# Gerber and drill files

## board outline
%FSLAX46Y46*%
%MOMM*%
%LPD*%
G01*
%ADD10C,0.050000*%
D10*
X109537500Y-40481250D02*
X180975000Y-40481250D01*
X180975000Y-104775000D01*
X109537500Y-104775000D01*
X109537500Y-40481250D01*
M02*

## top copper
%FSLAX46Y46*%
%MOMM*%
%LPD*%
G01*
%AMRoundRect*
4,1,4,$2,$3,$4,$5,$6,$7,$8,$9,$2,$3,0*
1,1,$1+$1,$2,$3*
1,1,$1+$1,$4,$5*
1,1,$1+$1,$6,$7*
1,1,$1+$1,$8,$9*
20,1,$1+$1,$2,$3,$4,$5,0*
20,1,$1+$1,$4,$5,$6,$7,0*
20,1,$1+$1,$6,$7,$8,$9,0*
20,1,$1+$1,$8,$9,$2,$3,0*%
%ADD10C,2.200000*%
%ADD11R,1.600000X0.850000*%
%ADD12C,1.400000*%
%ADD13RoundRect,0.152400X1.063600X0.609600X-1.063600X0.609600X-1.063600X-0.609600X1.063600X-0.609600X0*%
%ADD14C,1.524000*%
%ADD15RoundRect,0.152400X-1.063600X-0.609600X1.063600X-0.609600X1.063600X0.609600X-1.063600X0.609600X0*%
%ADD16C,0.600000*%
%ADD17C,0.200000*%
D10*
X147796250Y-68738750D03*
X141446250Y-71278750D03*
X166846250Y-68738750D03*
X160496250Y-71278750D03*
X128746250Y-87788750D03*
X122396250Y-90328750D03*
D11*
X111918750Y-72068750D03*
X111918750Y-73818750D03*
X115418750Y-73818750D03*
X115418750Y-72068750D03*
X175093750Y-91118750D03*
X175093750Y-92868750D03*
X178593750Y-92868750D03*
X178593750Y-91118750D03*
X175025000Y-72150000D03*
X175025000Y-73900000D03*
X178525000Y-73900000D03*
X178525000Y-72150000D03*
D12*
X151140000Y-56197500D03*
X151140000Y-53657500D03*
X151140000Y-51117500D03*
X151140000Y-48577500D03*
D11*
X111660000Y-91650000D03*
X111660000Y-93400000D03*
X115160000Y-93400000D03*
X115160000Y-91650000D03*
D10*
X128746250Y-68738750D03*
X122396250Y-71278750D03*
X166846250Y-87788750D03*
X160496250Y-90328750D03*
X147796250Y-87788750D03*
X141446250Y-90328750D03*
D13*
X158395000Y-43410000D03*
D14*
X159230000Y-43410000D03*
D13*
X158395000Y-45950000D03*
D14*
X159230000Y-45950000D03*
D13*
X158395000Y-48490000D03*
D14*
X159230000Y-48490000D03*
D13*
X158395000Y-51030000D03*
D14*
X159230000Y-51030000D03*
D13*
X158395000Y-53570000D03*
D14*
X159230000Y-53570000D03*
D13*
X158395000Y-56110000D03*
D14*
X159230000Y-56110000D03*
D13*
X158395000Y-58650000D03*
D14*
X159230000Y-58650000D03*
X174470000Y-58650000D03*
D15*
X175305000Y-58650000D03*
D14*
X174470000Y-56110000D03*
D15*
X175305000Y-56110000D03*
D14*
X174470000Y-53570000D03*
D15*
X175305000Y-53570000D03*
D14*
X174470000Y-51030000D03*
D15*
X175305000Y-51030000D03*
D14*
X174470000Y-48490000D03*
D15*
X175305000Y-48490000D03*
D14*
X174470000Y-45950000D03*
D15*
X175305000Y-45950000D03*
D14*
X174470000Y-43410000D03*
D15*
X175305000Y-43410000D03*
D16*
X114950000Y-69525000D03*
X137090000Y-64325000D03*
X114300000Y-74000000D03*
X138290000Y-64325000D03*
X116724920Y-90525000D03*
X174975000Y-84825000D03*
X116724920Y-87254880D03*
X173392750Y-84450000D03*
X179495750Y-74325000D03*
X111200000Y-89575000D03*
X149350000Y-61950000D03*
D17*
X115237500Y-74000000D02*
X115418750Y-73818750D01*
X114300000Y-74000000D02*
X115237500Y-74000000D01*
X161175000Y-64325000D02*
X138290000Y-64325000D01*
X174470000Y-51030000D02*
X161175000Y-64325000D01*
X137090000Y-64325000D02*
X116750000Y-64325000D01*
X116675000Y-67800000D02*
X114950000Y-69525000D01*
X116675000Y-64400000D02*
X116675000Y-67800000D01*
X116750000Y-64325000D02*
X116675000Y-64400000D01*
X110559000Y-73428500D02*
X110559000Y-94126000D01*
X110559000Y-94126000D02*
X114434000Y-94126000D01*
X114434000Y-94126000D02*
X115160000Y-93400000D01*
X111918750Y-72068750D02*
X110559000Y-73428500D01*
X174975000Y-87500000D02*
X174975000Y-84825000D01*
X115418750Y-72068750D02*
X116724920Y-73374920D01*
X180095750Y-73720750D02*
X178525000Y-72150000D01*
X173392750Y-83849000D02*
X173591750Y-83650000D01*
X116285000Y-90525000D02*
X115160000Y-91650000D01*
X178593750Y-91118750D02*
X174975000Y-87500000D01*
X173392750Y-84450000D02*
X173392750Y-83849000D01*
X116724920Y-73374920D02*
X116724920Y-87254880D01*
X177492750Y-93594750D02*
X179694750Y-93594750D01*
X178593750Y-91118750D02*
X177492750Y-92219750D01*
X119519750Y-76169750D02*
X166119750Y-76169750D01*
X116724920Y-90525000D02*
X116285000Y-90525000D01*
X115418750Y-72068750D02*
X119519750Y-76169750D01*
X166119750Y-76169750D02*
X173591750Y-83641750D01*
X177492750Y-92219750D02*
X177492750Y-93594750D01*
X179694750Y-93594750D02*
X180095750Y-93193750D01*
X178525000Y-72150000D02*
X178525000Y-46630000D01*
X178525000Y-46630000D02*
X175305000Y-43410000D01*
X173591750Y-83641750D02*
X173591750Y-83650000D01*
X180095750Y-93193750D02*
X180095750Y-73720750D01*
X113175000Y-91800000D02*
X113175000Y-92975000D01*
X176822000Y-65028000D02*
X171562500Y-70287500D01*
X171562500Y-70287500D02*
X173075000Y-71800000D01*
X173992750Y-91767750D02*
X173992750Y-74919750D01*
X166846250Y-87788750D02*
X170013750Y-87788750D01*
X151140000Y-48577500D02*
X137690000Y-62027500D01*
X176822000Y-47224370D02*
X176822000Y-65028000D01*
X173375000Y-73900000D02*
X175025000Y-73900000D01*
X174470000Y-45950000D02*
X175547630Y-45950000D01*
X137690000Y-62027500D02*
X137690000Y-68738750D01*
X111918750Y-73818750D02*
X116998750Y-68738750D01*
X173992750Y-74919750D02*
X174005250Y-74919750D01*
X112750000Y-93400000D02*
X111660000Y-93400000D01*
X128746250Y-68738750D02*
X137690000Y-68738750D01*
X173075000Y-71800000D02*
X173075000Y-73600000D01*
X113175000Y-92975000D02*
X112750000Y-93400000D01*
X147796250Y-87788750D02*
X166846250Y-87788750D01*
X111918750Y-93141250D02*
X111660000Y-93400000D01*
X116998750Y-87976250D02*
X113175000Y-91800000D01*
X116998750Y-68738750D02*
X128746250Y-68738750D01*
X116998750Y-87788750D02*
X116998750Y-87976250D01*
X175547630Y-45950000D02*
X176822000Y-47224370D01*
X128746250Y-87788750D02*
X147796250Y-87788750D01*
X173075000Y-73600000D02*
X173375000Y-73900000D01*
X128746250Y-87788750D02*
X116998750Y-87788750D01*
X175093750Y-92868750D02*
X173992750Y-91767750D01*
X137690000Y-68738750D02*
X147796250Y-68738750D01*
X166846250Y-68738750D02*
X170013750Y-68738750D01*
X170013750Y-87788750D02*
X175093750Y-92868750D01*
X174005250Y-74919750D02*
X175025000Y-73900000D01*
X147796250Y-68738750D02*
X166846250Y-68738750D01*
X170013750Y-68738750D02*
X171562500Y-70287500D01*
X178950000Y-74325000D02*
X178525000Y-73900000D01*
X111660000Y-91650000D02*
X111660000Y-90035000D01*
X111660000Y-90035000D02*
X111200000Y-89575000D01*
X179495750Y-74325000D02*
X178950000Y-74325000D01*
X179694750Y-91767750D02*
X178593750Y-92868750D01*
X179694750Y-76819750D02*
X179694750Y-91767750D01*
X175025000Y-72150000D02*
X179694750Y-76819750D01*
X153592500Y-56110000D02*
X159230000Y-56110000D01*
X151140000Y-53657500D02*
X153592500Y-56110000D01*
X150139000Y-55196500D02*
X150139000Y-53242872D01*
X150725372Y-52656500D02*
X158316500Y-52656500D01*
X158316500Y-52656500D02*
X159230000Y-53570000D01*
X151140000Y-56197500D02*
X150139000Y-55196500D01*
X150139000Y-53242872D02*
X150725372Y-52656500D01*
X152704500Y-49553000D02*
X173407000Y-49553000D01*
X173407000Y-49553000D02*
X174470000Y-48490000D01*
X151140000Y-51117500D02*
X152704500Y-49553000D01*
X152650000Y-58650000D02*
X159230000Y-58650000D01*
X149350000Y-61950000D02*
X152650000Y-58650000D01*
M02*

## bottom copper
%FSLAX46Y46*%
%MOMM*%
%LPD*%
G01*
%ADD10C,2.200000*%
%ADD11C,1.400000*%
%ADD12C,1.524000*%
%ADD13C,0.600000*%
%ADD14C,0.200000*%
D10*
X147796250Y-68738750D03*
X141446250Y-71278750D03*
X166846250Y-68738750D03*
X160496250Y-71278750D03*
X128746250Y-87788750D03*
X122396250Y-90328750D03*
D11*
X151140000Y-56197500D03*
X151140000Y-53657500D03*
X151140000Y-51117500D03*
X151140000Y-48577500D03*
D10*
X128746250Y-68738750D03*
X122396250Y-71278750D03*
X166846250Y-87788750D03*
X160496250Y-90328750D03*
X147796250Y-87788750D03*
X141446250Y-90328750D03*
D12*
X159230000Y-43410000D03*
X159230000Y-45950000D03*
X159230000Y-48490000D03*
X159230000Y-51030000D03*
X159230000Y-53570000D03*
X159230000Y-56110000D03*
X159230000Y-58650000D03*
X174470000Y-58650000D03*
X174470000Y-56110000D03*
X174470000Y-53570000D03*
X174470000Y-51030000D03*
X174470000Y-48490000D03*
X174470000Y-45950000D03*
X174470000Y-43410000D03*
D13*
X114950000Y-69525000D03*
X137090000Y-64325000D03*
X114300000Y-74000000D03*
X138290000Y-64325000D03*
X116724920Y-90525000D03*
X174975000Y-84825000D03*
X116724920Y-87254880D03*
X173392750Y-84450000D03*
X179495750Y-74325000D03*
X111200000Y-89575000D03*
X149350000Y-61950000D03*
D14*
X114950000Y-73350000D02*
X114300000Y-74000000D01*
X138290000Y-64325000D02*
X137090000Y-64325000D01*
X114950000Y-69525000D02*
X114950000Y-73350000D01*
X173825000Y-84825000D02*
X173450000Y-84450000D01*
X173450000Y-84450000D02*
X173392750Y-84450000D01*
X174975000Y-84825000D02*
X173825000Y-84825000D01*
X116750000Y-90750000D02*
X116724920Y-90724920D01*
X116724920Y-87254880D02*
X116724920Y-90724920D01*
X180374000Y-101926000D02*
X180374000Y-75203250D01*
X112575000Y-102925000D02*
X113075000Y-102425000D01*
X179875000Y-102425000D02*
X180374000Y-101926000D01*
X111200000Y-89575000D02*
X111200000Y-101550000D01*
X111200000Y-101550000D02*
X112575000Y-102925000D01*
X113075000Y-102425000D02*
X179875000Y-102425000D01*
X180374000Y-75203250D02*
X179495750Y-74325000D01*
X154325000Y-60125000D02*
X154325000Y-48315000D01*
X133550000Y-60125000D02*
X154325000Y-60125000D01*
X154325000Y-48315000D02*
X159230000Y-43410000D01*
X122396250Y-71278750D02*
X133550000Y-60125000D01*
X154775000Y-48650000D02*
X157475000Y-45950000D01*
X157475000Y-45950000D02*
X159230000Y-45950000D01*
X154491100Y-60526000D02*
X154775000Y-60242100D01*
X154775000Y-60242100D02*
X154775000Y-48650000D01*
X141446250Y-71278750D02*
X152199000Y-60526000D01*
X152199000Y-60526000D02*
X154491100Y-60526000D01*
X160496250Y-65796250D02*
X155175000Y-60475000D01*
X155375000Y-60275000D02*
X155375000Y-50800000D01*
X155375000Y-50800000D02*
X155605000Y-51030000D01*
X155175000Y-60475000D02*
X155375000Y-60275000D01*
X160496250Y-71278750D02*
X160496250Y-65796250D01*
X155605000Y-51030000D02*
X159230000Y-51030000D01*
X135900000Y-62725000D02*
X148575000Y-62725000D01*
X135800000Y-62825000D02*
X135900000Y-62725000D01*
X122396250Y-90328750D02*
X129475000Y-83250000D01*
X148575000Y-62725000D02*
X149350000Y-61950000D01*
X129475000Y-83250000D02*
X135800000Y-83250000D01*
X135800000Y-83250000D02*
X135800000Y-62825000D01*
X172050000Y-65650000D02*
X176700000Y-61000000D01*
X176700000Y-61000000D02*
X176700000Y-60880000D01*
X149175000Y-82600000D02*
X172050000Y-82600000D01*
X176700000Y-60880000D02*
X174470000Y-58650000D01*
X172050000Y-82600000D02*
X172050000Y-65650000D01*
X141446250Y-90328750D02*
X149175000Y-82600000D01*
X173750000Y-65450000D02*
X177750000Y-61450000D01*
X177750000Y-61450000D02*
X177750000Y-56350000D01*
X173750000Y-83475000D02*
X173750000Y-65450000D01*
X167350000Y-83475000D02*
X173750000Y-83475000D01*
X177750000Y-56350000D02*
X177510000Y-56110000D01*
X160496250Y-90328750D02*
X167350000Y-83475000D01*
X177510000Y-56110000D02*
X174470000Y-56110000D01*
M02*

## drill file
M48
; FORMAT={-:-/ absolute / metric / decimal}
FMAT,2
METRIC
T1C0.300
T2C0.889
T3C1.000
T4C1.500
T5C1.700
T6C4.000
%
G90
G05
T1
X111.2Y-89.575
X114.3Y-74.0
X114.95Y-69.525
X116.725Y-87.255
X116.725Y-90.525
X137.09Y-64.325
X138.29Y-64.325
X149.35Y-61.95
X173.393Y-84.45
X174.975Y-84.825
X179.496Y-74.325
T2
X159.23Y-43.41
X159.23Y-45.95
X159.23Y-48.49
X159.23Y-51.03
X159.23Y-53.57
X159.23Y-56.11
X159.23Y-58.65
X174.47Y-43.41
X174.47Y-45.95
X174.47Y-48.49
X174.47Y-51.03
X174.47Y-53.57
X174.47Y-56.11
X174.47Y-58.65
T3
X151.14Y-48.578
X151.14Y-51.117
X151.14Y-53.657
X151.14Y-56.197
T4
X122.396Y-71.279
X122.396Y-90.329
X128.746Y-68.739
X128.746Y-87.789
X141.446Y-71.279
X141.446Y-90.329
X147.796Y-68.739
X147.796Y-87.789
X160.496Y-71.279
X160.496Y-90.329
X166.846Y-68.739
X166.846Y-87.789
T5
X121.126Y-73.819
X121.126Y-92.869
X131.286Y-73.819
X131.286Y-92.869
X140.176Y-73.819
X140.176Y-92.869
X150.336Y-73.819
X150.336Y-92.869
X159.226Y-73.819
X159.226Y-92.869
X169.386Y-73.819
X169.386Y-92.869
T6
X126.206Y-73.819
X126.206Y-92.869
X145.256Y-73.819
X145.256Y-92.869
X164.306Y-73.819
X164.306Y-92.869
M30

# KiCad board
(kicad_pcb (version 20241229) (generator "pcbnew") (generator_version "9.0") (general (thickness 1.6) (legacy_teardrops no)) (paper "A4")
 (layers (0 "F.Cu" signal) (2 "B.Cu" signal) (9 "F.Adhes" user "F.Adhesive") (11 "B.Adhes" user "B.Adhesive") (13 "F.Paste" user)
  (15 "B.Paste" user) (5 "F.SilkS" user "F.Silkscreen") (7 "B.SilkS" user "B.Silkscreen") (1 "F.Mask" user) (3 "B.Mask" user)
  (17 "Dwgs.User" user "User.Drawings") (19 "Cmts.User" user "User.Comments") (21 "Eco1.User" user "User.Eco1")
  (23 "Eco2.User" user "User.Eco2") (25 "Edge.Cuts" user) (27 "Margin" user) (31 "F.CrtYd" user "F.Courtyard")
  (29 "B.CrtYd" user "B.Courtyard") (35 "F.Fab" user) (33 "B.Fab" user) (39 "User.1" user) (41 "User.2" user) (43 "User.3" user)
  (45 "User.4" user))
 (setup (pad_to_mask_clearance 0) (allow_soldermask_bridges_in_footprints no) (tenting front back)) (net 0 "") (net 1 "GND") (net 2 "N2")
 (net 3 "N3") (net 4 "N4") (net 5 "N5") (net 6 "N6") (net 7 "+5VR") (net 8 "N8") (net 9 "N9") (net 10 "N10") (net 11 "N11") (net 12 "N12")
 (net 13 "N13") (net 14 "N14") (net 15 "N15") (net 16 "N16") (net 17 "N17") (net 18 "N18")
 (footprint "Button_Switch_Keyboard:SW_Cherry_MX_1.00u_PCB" (layer "F.Cu") (at 147.79625 68.73875)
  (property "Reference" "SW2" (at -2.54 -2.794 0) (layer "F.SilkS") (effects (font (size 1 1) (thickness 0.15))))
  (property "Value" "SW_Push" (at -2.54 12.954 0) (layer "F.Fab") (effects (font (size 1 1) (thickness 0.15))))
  (pad "" np_thru_hole circle (at -7.62 5.08) (size 1.7 1.7) (drill 1.7) (layers "*.Cu" "*.Mask"))
  (pad "" np_thru_hole circle (at -2.54 5.08) (size 4 4) (drill 4) (layers "*.Cu" "*.Mask"))
  (pad "" np_thru_hole circle (at 2.54 5.08) (size 1.7 1.7) (drill 1.7) (layers "*.Cu" "*.Mask"))
  (pad "1" thru_hole circle (at 0 0) (size 2.2 2.2) (drill 1.5) (layers "*.Cu" "*.Mask") (remove_unused_layers no) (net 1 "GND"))
  (pad "2" thru_hole circle (at -6.35 2.54) (size 2.2 2.2) (drill 1.5) (layers "*.Cu" "*.Mask") (remove_unused_layers no) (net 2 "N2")))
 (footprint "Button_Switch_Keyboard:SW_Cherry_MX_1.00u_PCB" (layer "F.Cu") (at 166.84625 68.73875)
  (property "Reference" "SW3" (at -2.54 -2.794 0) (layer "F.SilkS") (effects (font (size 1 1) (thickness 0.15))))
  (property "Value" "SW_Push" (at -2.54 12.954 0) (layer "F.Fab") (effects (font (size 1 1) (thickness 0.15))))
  (pad "" np_thru_hole circle (at -7.62 5.08) (size 1.7 1.7) (drill 1.7) (layers "*.Cu" "*.Mask"))
  (pad "" np_thru_hole circle (at -2.54 5.08) (size 4 4) (drill 4) (layers "*.Cu" "*.Mask"))
  (pad "" np_thru_hole circle (at 2.54 5.08) (size 1.7 1.7) (drill 1.7) (layers "*.Cu" "*.Mask"))
  (pad "1" thru_hole circle (at 0 0) (size 2.2 2.2) (drill 1.5) (layers "*.Cu" "*.Mask") (remove_unused_layers no) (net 1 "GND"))
  (pad "2" thru_hole circle (at -6.35 2.54) (size 2.2 2.2) (drill 1.5) (layers "*.Cu" "*.Mask") (remove_unused_layers no) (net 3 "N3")))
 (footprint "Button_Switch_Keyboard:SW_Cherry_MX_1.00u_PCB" (layer "F.Cu") (at 128.74625 87.78875)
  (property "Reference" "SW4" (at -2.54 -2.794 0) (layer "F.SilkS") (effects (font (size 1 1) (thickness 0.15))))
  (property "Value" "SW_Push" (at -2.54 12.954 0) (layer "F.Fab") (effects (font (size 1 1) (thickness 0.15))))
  (pad "" np_thru_hole circle (at -7.62 5.08) (size 1.7 1.7) (drill 1.7) (layers "*.Cu" "*.Mask"))
  (pad "" np_thru_hole circle (at -2.54 5.08) (size 4 4) (drill 4) (layers "*.Cu" "*.Mask"))
  (pad "" np_thru_hole circle (at 2.54 5.08) (size 1.7 1.7) (drill 1.7) (layers "*.Cu" "*.Mask"))
  (pad "1" thru_hole circle (at 0 0) (size 2.2 2.2) (drill 1.5) (layers "*.Cu" "*.Mask") (remove_unused_layers no) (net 1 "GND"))
  (pad "2" thru_hole circle (at -6.35 2.54) (size 2.2 2.2) (drill 1.5) (layers "*.Cu" "*.Mask") (remove_unused_layers no) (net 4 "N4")))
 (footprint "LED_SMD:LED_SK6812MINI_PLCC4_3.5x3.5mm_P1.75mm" (layer "F.Cu") (at 113.66875 72.94375)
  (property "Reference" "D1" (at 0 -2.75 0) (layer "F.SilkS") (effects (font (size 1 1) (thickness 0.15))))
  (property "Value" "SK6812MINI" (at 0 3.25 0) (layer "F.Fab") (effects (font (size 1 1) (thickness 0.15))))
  (pad "1" smd rect (at -1.75 -0.875) (size 1.6 0.85) (layers "F.Cu" "F.Mask" "F.Paste") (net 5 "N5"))
  (pad "2" smd rect (at -1.75 0.875) (size 1.6 0.85) (layers "F.Cu" "F.Mask" "F.Paste") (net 1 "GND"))
  (pad "3" smd rect (at 1.75 0.875) (size 1.6 0.85) (layers "F.Cu" "F.Mask" "F.Paste") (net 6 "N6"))
  (pad "4" smd rect (at 1.75 -0.875) (size 1.6 0.85) (layers "F.Cu" "F.Mask" "F.Paste") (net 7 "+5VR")))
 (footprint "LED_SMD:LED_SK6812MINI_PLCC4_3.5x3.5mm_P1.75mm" (layer "F.Cu") (at 176.84375 91.99375)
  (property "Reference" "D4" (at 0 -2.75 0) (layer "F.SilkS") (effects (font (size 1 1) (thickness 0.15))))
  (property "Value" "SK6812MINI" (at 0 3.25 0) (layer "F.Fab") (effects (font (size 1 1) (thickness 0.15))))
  (pad "1" smd rect (at -1.75 -0.875) (size 1.6 0.85) (layers "F.Cu" "F.Mask" "F.Paste") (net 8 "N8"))
  (pad "2" smd rect (at -1.75 0.875) (size 1.6 0.85) (layers "F.Cu" "F.Mask" "F.Paste") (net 1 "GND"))
  (pad "3" smd rect (at 1.75 0.875) (size 1.6 0.85) (layers "F.Cu" "F.Mask" "F.Paste") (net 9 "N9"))
  (pad "4" smd rect (at 1.75 -0.875) (size 1.6 0.85) (layers "F.Cu" "F.Mask" "F.Paste") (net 7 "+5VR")))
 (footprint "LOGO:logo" (layer "F.Cu") (at 143.875 81.625)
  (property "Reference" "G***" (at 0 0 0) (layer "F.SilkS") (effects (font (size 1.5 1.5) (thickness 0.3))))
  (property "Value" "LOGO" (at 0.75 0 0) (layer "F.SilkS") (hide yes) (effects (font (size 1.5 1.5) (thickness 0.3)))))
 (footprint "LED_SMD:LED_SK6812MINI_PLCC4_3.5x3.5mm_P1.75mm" (layer "F.Cu") (at 176.775 73.025)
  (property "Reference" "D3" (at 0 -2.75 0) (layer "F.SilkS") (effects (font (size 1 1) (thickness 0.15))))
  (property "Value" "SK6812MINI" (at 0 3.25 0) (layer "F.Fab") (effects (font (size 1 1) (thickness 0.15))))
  (pad "1" smd rect (at -1.75 -0.875) (size 1.6 0.85) (layers "F.Cu" "F.Mask" "F.Paste") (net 9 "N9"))
  (pad "2" smd rect (at -1.75 0.875) (size 1.6 0.85) (layers "F.Cu" "F.Mask" "F.Paste") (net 1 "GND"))
  (pad "3" smd rect (at 1.75 0.875) (size 1.6 0.85) (layers "F.Cu" "F.Mask" "F.Paste") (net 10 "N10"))
  (pad "4" smd rect (at 1.75 -0.875) (size 1.6 0.85) (layers "F.Cu" "F.Mask" "F.Paste") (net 7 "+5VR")))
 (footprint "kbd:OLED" (layer "F.Cu") (at 151.14 52.3875 90)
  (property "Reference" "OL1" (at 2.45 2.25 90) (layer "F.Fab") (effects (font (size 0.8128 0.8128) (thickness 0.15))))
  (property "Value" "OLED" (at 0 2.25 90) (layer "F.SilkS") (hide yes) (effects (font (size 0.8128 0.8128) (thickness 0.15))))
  (pad "1" thru_hole circle (at -3.81 0 90) (size 1.4 1.4) (drill 1) (layers "*.Cu" "*.Mask") (remove_unused_layers no) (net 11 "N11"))
  (pad "2" thru_hole circle (at -1.27 0 90) (size 1.4 1.4) (drill 1) (layers "*.Cu" "*.Mask") (remove_unused_layers no) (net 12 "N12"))
  (pad "3" thru_hole circle (at 1.27 0 90) (size 1.4 1.4) (drill 1) (layers "*.Cu" "*.Mask") (remove_unused_layers no) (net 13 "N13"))
  (pad "4" thru_hole circle (at 3.81 0 90) (size 1.4 1.4) (drill 1) (layers "*.Cu" "*.Mask") (remove_unused_layers no) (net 1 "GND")))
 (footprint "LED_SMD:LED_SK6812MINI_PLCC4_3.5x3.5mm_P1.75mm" (layer "F.Cu") (at 113.41 92.525)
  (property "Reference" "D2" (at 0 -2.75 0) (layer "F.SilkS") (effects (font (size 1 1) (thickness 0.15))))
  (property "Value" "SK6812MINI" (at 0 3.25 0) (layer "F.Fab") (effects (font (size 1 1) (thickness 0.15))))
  (pad "1" smd rect (at -1.75 -0.875) (size 1.6 0.85) (layers "F.Cu" "F.Mask" "F.Paste") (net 10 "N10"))
  (pad "2" smd rect (at -1.75 0.875) (size 1.6 0.85) (layers "F.Cu" "F.Mask" "F.Paste") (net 1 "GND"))
  (pad "3" smd rect (at 1.75 0.875) (size 1.6 0.85) (layers "F.Cu" "F.Mask" "F.Paste") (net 5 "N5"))
  (pad "4" smd rect (at 1.75 -0.875) (size 1.6 0.85) (layers "F.Cu" "F.Mask" "F.Paste") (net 7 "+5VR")))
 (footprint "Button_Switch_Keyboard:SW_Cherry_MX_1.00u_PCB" (layer "F.Cu") (at 128.74625 68.73875)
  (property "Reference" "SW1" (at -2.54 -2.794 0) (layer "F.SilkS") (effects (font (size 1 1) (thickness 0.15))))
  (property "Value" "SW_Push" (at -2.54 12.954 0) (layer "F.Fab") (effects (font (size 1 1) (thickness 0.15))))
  (pad "" np_thru_hole circle (at -7.62 5.08) (size 1.7 1.7) (drill 1.7) (layers "*.Cu" "*.Mask"))
  (pad "" np_thru_hole circle (at -2.54 5.08) (size 4 4) (drill 4) (layers "*.Cu" "*.Mask"))
  (pad "" np_thru_hole circle (at 2.54 5.08) (size 1.7 1.7) (drill 1.7) (layers "*.Cu" "*.Mask"))
  (pad "1" thru_hole circle (at 0 0) (size 2.2 2.2) (drill 1.5) (layers "*.Cu" "*.Mask") (remove_unused_layers no) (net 1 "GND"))
  (pad "2" thru_hole circle (at -6.35 2.54) (size 2.2 2.2) (drill 1.5) (layers "*.Cu" "*.Mask") (remove_unused_layers no) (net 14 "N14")))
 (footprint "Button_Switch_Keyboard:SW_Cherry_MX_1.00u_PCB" (layer "F.Cu") (at 166.84625 87.78875)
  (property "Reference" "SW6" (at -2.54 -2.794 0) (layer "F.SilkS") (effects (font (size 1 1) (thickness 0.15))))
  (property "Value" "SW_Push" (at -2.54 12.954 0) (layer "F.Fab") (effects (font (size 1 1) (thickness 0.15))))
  (pad "" np_thru_hole circle (at -7.62 5.08) (size 1.7 1.7) (drill 1.7) (layers "*.Cu" "*.Mask"))
  (pad "" np_thru_hole circle (at -2.54 5.08) (size 4 4) (drill 4) (layers "*.Cu" "*.Mask"))
  (pad "" np_thru_hole circle (at 2.54 5.08) (size 1.7 1.7) (drill 1.7) (layers "*.Cu" "*.Mask"))
  (pad "1" thru_hole circle (at 0 0) (size 2.2 2.2) (drill 1.5) (layers "*.Cu" "*.Mask") (remove_unused_layers no) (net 1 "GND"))
  (pad "2" thru_hole circle (at -6.35 2.54) (size 2.2 2.2) (drill 1.5) (layers "*.Cu" "*.Mask") (remove_unused_layers no) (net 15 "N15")))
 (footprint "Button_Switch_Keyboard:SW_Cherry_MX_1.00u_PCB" (layer "F.Cu") (at 147.79625 87.78875)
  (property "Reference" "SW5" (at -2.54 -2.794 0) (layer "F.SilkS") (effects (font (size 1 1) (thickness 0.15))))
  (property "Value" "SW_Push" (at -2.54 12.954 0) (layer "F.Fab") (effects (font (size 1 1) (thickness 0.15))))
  (pad "" np_thru_hole circle (at -7.62 5.08) (size 1.7 1.7) (drill 1.7) (layers "*.Cu" "*.Mask"))
  (pad "" np_thru_hole circle (at -2.54 5.08) (size 4 4) (drill 4) (layers "*.Cu" "*.Mask"))
  (pad "" np_thru_hole circle (at 2.54 5.08) (size 1.7 1.7) (drill 1.7) (layers "*.Cu" "*.Mask"))
  (pad "1" thru_hole circle (at 0 0) (size 2.2 2.2) (drill 1.5) (layers "*.Cu" "*.Mask") (remove_unused_layers no) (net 1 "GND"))
  (pad "2" thru_hole circle (at -6.35 2.54) (size 2.2 2.2) (drill 1.5) (layers "*.Cu" "*.Mask") (remove_unused_layers no) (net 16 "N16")))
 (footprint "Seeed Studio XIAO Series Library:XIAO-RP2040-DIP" (layer "F.Cu") (at 166.85 51.03)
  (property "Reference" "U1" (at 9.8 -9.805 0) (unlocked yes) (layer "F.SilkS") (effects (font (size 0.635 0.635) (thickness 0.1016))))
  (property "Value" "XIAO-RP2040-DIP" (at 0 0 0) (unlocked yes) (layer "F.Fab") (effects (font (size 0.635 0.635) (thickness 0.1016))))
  (pad "1" smd roundrect (at -8.455 -7.62 180) (size 2.432 1.524) (layers "F.Cu" "F.Mask") (roundrect_rratio 0.1) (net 14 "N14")
   (thermal_bridge_angle 45))
  (pad "1" thru_hole circle (at -7.62 -7.62 180) (size 1.524 1.524) (drill 0.889) (layers "*.Cu" "*.Mask") (remove_unused_layers no)
   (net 14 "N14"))
  (pad "2" smd roundrect (at -8.455 -5.08 180) (size 2.432 1.524) (layers "F.Cu" "F.Mask") (roundrect_rratio 0.1) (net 2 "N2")
   (thermal_bridge_angle 45))
  (pad "2" thru_hole circle (at -7.62 -5.08 180) (size 1.524 1.524) (drill 0.889) (layers "*.Cu" "*.Mask") (remove_unused_layers no)
   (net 2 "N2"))
  (pad "3" smd roundrect (at -8.455 -2.54 180) (size 2.432 1.524) (layers "F.Cu" "F.Mask") (roundrect_rratio 0.1) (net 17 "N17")
   (thermal_bridge_angle 45))
  (pad "3" thru_hole circle (at -7.62 -2.54 180) (size 1.524 1.524) (drill 0.889) (layers "*.Cu" "*.Mask") (remove_unused_layers no)
   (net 17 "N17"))
  (pad "4" smd roundrect (at -8.455 0 180) (size 2.432 1.524) (layers "F.Cu" "F.Mask") (roundrect_rratio 0.1) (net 3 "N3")
   (thermal_bridge_angle 45))
  (pad "4" thru_hole circle (at -7.62 0 180) (size 1.524 1.524) (drill 0.889) (layers "*.Cu" "*.Mask") (remove_unused_layers no)
   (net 3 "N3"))
  (pad "5" smd roundrect (at -8.455 2.54 180) (size 2.432 1.524) (layers "F.Cu" "F.Mask") (roundrect_rratio 0.1) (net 11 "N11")
   (thermal_bridge_angle 45))
  (pad "5" thru_hole circle (at -7.62 2.54 180) (size 1.524 1.524) (drill 0.889) (layers "*.Cu" "*.Mask") (remove_unused_layers no)
   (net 11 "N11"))
  (pad "6" smd roundrect (at -8.455 5.08 180) (size 2.432 1.524) (layers "F.Cu" "F.Mask") (roundrect_rratio 0.1) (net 12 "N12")
   (thermal_bridge_angle 45))
  (pad "6" thru_hole circle (at -7.62 5.08 180) (size 1.524 1.524) (drill 0.889) (layers "*.Cu" "*.Mask") (remove_unused_layers no)
   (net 12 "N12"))
  (pad "7" smd roundrect (at -8.455 7.62 180) (size 2.432 1.524) (layers "F.Cu" "F.Mask") (roundrect_rratio 0.1) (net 4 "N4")
   (thermal_bridge_angle 45))
  (pad "7" thru_hole circle (at -7.62 7.62 180) (size 1.524 1.524) (drill 0.889) (layers "*.Cu" "*.Mask") (remove_unused_layers no)
   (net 4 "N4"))
  (pad "8" thru_hole circle (at 7.62 7.62) (size 1.524 1.524) (drill 0.889) (layers "*.Cu" "*.Mask") (remove_unused_layers no)
   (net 16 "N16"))
  (pad "8" smd roundrect (at 8.455 7.62) (size 2.432 1.524) (layers "F.Cu" "F.Mask") (roundrect_rratio 0.1) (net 16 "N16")
   (thermal_bridge_angle 45))
  (pad "9" thru_hole circle (at 7.62 5.08) (size 1.524 1.524) (drill 0.889) (layers "*.Cu" "*.Mask") (remove_unused_layers no)
   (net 15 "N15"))
  (pad "9" smd roundrect (at 8.455 5.08) (size 2.432 1.524) (layers "F.Cu" "F.Mask") (roundrect_rratio 0.1) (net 15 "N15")
   (thermal_bridge_angle 45))
  (pad "10" thru_hole circle (at 7.62 2.54) (size 1.524 1.524) (drill 0.889) (layers "*.Cu" "*.Mask") (remove_unused_layers no)
   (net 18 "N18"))
  (pad "10" smd roundrect (at 8.455 2.54) (size 2.432 1.524) (layers "F.Cu" "F.Mask") (roundrect_rratio 0.1) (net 18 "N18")
   (thermal_bridge_angle 45))
  (pad "11" thru_hole circle (at 7.62 0) (size 1.524 1.524) (drill 0.889) (layers "*.Cu" "*.Mask") (remove_unused_layers no) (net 6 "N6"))
  (pad "11" smd roundrect (at 8.455 0) (size 2.432 1.524) (layers "F.Cu" "F.Mask") (roundrect_rratio 0.1) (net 6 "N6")
   (thermal_bridge_angle 45))
  (pad "12" thru_hole circle (at 7.62 -2.54) (size 1.524 1.524) (drill 0.889) (layers "*.Cu" "*.Mask") (remove_unused_layers no)
   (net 13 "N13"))
  (pad "12" smd roundrect (at 8.455 -2.54) (size 2.432 1.524) (layers "F.Cu" "F.Mask") (roundrect_rratio 0.1) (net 13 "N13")
   (thermal_bridge_angle 45))
  (pad "13" thru_hole circle (at 7.62 -5.08) (size 1.524 1.524) (drill 0.889) (layers "*.Cu" "*.Mask") (remove_unused_layers no)
   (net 1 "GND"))
  (pad "13" smd roundrect (at 8.455 -5.08) (size 2.432 1.524) (layers "F.Cu" "F.Mask") (roundrect_rratio 0.1) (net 1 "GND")
   (thermal_bridge_angle 45))
  (pad "14" thru_hole circle (at 7.62 -7.62) (size 1.524 1.524) (drill 0.889) (layers "*.Cu" "*.Mask") (remove_unused_layers no)
   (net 7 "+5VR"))
  (pad "14" smd roundrect (at 8.455 -7.62) (size 2.432 1.524) (layers "F.Cu" "F.Mask") (roundrect_rratio 0.1) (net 7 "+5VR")
   (thermal_bridge_angle 45)))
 (gr_rect (start 109.5375 40.48125) (end 180.975 104.775) (stroke (width 0.05) (type default)) (fill no) (layer "Edge.Cuts"))
 (segment (start 115.2375 74) (end 115.41875 73.81875) (width 0.2) (layer "F.Cu") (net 6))
 (segment (start 114.3 74) (end 115.2375 74) (width 0.2) (layer "F.Cu") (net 6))
 (segment (start 161.175 64.325) (end 138.29 64.325) (width 0.2) (layer "F.Cu") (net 6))
 (segment (start 174.47 51.03) (end 161.175 64.325) (width 0.2) (layer "F.Cu") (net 6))
 (segment (start 137.09 64.325) (end 116.75 64.325) (width 0.2) (layer "F.Cu") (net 6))
 (segment (start 116.675 67.8) (end 114.95 69.525) (width 0.2) (layer "F.Cu") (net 6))
 (segment (start 116.675 64.4) (end 116.675 67.8) (width 0.2) (layer "F.Cu") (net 6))
 (segment (start 116.75 64.325) (end 116.675 64.4) (width 0.2) (layer "F.Cu") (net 6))
 (via (at 114.95 69.525) (size 0.6) (drill 0.3) (layers "F.Cu" "B.Cu") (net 6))
 (via (at 137.09 64.325) (size 0.6) (drill 0.3) (layers "F.Cu" "B.Cu") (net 6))
 (via (at 114.3 74) (size 0.6) (drill 0.3) (layers "F.Cu" "B.Cu") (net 6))
 (via (at 138.29 64.325) (size 0.6) (drill 0.3) (layers "F.Cu" "B.Cu") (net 6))
 (segment (start 114.95 73.35) (end 114.3 74) (width 0.2) (layer "B.Cu") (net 6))
 (segment (start 138.29 64.325) (end 137.09 64.325) (width 0.2) (layer "B.Cu") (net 6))
 (segment (start 114.95 69.525) (end 114.95 73.35) (width 0.2) (layer "B.Cu") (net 6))
 (segment (start 110.559 73.4285) (end 110.559 94.126) (width 0.2) (layer "F.Cu") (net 5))
 (segment (start 110.559 94.126) (end 114.434 94.126) (width 0.2) (layer "F.Cu") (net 5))
 (segment (start 114.434 94.126) (end 115.16 93.4) (width 0.2) (layer "F.Cu") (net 5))
 (segment (start 111.91875 72.06875) (end 110.559 73.4285) (width 0.2) (layer "F.Cu") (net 5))
 (segment (start 174.975 87.5) (end 174.975 84.825) (width 0.2) (layer "F.Cu") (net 7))
 (segment (start 115.41875 72.06875) (end 116.72492 73.37492) (width 0.2) (layer "F.Cu") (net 7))
 (segment (start 180.09575 73.72075) (end 178.525 72.15) (width 0.2) (layer "F.Cu") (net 7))
 (segment (start 173.39275 83.849) (end 173.59175 83.65) (width 0.2) (layer "F.Cu") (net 7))
 (segment (start 116.285 90.525) (end 115.16 91.65) (width 0.2) (layer "F.Cu") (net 7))
 (segment (start 178.59375 91.11875) (end 174.975 87.5) (width 0.2) (layer "F.Cu") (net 7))
 (segment (start 173.39275 84.45) (end 173.39275 83.849) (width 0.2) (layer "F.Cu") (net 7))
 (segment (start 116.72492 73.37492) (end 116.72492 87.25488) (width 0.2) (layer "F.Cu") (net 7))
 (segment (start 177.49275 93.59475) (end 179.69475 93.59475) (width 0.2) (layer "F.Cu") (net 7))
 (segment (start 178.59375 91.11875) (end 177.49275 92.21975) (width 0.2) (layer "F.Cu") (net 7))
 (segment (start 119.51975 76.16975) (end 166.11975 76.16975) (width 0.2) (layer "F.Cu") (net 7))
 (segment (start 116.72492 90.525) (end 116.285 90.525) (width 0.2) (layer "F.Cu") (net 7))
 (segment (start 115.41875 72.06875) (end 119.51975 76.16975) (width 0.2) (layer "F.Cu") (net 7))
 (segment (start 166.11975 76.16975) (end 173.59175 83.64175) (width 0.2) (layer "F.Cu") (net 7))
 (segment (start 177.49275 92.21975) (end 177.49275 93.59475) (width 0.2) (layer "F.Cu") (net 7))
 (segment (start 179.69475 93.59475) (end 180.09575 93.19375) (width 0.2) (layer "F.Cu") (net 7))
 (segment (start 178.525 72.15) (end 178.525 46.63) (width 0.2) (layer "F.Cu") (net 7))
 (segment (start 178.525 46.63) (end 175.305 43.41) (width 0.2) (layer "F.Cu") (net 7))
 (segment (start 173.59175 83.64175) (end 173.59175 83.65) (width 0.2) (layer "F.Cu") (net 7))
 (segment (start 180.09575 93.19375) (end 180.09575 73.72075) (width 0.2) (layer "F.Cu") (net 7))
 (via (at 116.72492 90.525) (size 0.6) (drill 0.3) (layers "F.Cu" "B.Cu") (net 7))
 (via (at 174.975 84.825) (size 0.6) (drill 0.3) (layers "F.Cu" "B.Cu") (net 7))
 (via (at 116.72492 87.25488) (size 0.6) (drill 0.3) (layers "F.Cu" "B.Cu") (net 7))
 (via (at 173.39275 84.45) (size 0.6) (drill 0.3) (layers "F.Cu" "B.Cu") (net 7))
 (segment (start 173.825 84.825) (end 173.45 84.45) (width 0.2) (layer "B.Cu") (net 7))
 (segment (start 173.45 84.45) (end 173.39275 84.45) (width 0.2) (layer "B.Cu") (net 7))
 (segment (start 174.975 84.825) (end 173.825 84.825) (width 0.2) (layer "B.Cu") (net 7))
 (segment (start 116.75 90.75) (end 116.72492 90.72492) (width 0.2) (layer "B.Cu") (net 7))
 (segment (start 116.72492 87.25488) (end 116.72492 90.72492) (width 0.2) (layer "B.Cu") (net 7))
 (segment (start 113.175 91.8) (end 113.175 92.975) (width 0.2) (layer "F.Cu") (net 1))
 (segment (start 176.822 65.028) (end 171.5625 70.2875) (width 0.2) (layer "F.Cu") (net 1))
 (segment (start 171.5625 70.2875) (end 173.075 71.8) (width 0.2) (layer "F.Cu") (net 1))
 (segment (start 173.99275 91.76775) (end 173.99275 74.91975) (width 0.2) (layer "F.Cu") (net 1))
 (segment (start 166.84625 87.78875) (end 170.01375 87.78875) (width 0.2) (layer "F.Cu") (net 1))
 (segment (start 151.14 48.5775) (end 137.69 62.0275) (width 0.2) (layer "F.Cu") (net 1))
 (segment (start 176.822 47.22437) (end 176.822 65.028) (width 0.2) (layer "F.Cu") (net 1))
 (segment (start 173.375 73.9) (end 175.025 73.9) (width 0.2) (layer "F.Cu") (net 1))
 (segment (start 174.47 45.95) (end 175.54763 45.95) (width 0.2) (layer "F.Cu") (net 1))
 (segment (start 137.69 62.0275) (end 137.69 68.73875) (width 0.2) (layer "F.Cu") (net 1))
 (segment (start 111.91875 73.81875) (end 116.99875 68.73875) (width 0.2) (layer "F.Cu") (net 1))
 (segment (start 173.99275 74.91975) (end 174.00525 74.91975) (width 0.2) (layer "F.Cu") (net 1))
 (segment (start 112.75 93.4) (end 111.66 93.4) (width 0.2) (layer "F.Cu") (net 1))
 (segment (start 128.74625 68.73875) (end 137.69 68.73875) (width 0.2) (layer "F.Cu") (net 1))
 (segment (start 173.075 71.8) (end 173.075 73.6) (width 0.2) (layer "F.Cu") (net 1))
 (segment (start 113.175 92.975) (end 112.75 93.4) (width 0.2) (layer "F.Cu") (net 1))
 (segment (start 147.79625 87.78875) (end 166.84625 87.78875) (width 0.2) (layer "F.Cu") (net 1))
 (segment (start 111.91875 93.14125) (end 111.66 93.4) (width 0.2) (layer "F.Cu") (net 1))
 (segment (start 116.99875 87.97625) (end 113.175 91.8) (width 0.2) (layer "F.Cu") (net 1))
 (segment (start 116.99875 68.73875) (end 128.74625 68.73875) (width 0.2) (layer "F.Cu") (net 1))
 (segment (start 116.99875 87.78875) (end 116.99875 87.97625) (width 0.2) (layer "F.Cu") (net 1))
 (segment (start 175.54763 45.95) (end 176.822 47.22437) (width 0.2) (layer "F.Cu") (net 1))
 (segment (start 128.74625 87.78875) (end 147.79625 87.78875) (width 0.2) (layer "F.Cu") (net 1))
 (segment (start 173.075 73.6) (end 173.375 73.9) (width 0.2) (layer "F.Cu") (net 1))
 (segment (start 128.74625 87.78875) (end 116.99875 87.78875) (width 0.2) (layer "F.Cu") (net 1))
 (segment (start 175.09375 92.86875) (end 173.99275 91.76775) (width 0.2) (layer "F.Cu") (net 1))
 (segment (start 137.69 68.73875) (end 147.79625 68.73875) (width 0.2) (layer "F.Cu") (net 1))
 (segment (start 166.84625 68.73875) (end 170.01375 68.73875) (width 0.2) (layer "F.Cu") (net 1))
 (segment (start 170.01375 87.78875) (end 175.09375 92.86875) (width 0.2) (layer "F.Cu") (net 1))
 (segment (start 174.00525 74.91975) (end 175.025 73.9) (width 0.2) (layer "F.Cu") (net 1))
 (segment (start 147.79625 68.73875) (end 166.84625 68.73875) (width 0.2) (layer "F.Cu") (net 1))
 (segment (start 170.01375 68.73875) (end 171.5625 70.2875) (width 0.2) (layer "F.Cu") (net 1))
 (segment (start 178.95 74.325) (end 178.525 73.9) (width 0.2) (layer "F.Cu") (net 10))
 (segment (start 111.66 91.65) (end 111.66 90.035) (width 0.2) (layer "F.Cu") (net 10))
 (segment (start 111.66 90.035) (end 111.2 89.575) (width 0.2) (layer "F.Cu") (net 10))
 (segment (start 179.49575 74.325) (end 178.95 74.325) (width 0.2) (layer "F.Cu") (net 10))
 (via (at 179.49575 74.325) (size 0.6) (drill 0.3) (layers "F.Cu" "B.Cu") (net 10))
 (via (at 111.2 89.575) (size 0.6) (drill 0.3) (layers "F.Cu" "B.Cu") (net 10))
 (segment (start 180.374 101.926) (end 180.374 75.20325) (width 0.2) (layer "B.Cu") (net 10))
 (segment (start 112.575 102.925) (end 113.075 102.425) (width 0.2) (layer "B.Cu") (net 10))
 (segment (start 179.875 102.425) (end 180.374 101.926) (width 0.2) (layer "B.Cu") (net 10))
 (segment (start 111.2 89.575) (end 111.2 101.55) (width 0.2) (layer "B.Cu") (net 10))
 (segment (start 111.2 101.55) (end 112.575 102.925) (width 0.2) (layer "B.Cu") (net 10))
 (segment (start 113.075 102.425) (end 179.875 102.425) (width 0.2) (layer "B.Cu") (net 10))
 (segment (start 180.374 75.20325) (end 179.49575 74.325) (width 0.2) (layer "B.Cu") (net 10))
 (segment (start 179.69475 91.76775) (end 178.59375 92.86875) (width 0.2) (layer "F.Cu") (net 9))
 (segment (start 179.69475 76.81975) (end 179.69475 91.76775) (width 0.2) (layer "F.Cu") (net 9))
 (segment (start 175.025 72.15) (end 179.69475 76.81975) (width 0.2) (layer "F.Cu") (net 9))
 (segment (start 153.5925 56.11) (end 159.23 56.11) (width 0.2) (layer "F.Cu") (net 12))
 (segment (start 151.14 53.6575) (end 153.5925 56.11) (width 0.2) (layer "F.Cu") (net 12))
 (segment (start 150.139 55.1965) (end 150.139 53.242872) (width 0.2) (layer "F.Cu") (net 11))
 (segment (start 150.725372 52.6565) (end 158.3165 52.6565) (width 0.2) (layer "F.Cu") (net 11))
 (segment (start 158.3165 52.6565) (end 159.23 53.57) (width 0.2) (layer "F.Cu") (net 11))
 (segment (start 151.14 56.1975) (end 150.139 55.1965) (width 0.2) (layer "F.Cu") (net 11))
 (segment (start 150.139 53.242872) (end 150.725372 52.6565) (width 0.2) (layer "F.Cu") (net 11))
 (segment (start 152.7045 49.553) (end 173.407 49.553) (width 0.2) (layer "F.Cu") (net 13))
 (segment (start 173.407 49.553) (end 174.47 48.49) (width 0.2) (layer "F.Cu") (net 13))
 (segment (start 151.14 51.1175) (end 152.7045 49.553) (width 0.2) (layer "F.Cu") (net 13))
 (segment (start 154.325 60.125) (end 154.325 48.315) (width 0.2) (layer "B.Cu") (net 14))
 (segment (start 133.55 60.125) (end 154.325 60.125) (width 0.2) (layer "B.Cu") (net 14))
 (segment (start 154.325 48.315) (end 159.23 43.41) (width 0.2) (layer "B.Cu") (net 14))
 (segment (start 122.39625 71.27875) (end 133.55 60.125) (width 0.2) (layer "B.Cu") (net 14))
 (segment (start 154.775 48.65) (end 157.475 45.95) (width 0.2) (layer "B.Cu") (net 2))
 (segment (start 157.475 45.95) (end 159.23 45.95) (width 0.2) (layer "B.Cu") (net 2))
 (segment (start 154.4911 60.526) (end 154.775 60.2421) (width 0.2) (layer "B.Cu") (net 2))
 (segment (start 154.775 60.2421) (end 154.775 48.65) (width 0.2) (layer "B.Cu") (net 2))
 (segment (start 141.44625 71.27875) (end 152.199 60.526) (width 0.2) (layer "B.Cu") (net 2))
 (segment (start 152.199 60.526) (end 154.4911 60.526) (width 0.2) (layer "B.Cu") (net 2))
 (segment (start 160.49625 65.79625) (end 155.175 60.475) (width 0.2) (layer "B.Cu") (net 3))
 (segment (start 155.375 60.275) (end 155.375 50.8) (width 0.2) (layer "B.Cu") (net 3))
 (segment (start 155.375 50.8) (end 155.605 51.03) (width 0.2) (layer "B.Cu") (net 3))
 (segment (start 155.175 60.475) (end 155.375 60.275) (width 0.2) (layer "B.Cu") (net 3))
 (segment (start 160.49625 71.27875) (end 160.49625 65.79625) (width 0.2) (layer "B.Cu") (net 3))
 (segment (start 155.605 51.03) (end 159.23 51.03) (width 0.2) (layer "B.Cu") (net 3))
 (segment (start 152.65 58.65) (end 159.23 58.65) (width 0.2) (layer "F.Cu") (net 4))
 (segment (start 149.35 61.95) (end 152.65 58.65) (width 0.2) (layer "F.Cu") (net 4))
 (via (at 149.35 61.95) (size 0.6) (drill 0.3) (layers "F.Cu" "B.Cu") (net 4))
 (segment (start 135.9 62.725) (end 148.575 62.725) (width 0.2) (layer "B.Cu") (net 4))
 (segment (start 135.8 62.825) (end 135.9 62.725) (width 0.2) (layer "B.Cu") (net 4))
 (segment (start 122.39625 90.32875) (end 129.475 83.25) (width 0.2) (layer "B.Cu") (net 4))
 (segment (start 148.575 62.725) (end 149.35 61.95) (width 0.2) (layer "B.Cu") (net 4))
 (segment (start 129.475 83.25) (end 135.8 83.25) (width 0.2) (layer "B.Cu") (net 4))
 (segment (start 135.8 83.25) (end 135.8 62.825) (width 0.2) (layer "B.Cu") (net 4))
 (segment (start 172.05 65.65) (end 176.7 61) (width 0.2) (layer "B.Cu") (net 16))
 (segment (start 176.7 61) (end 176.7 60.88) (width 0.2) (layer "B.Cu") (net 16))
 (segment (start 149.175 82.6) (end 172.05 82.6) (width 0.2) (layer "B.Cu") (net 16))
 (segment (start 176.7 60.88) (end 174.47 58.65) (width 0.2) (layer "B.Cu") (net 16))
 (segment (start 172.05 82.6) (end 172.05 65.65) (width 0.2) (layer "B.Cu") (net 16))
 (segment (start 141.44625 90.32875) (end 149.175 82.6) (width 0.2) (layer "B.Cu") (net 16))
 (segment (start 173.75 65.45) (end 177.75 61.45) (width 0.2) (layer "B.Cu") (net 15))
 (segment (start 177.75 61.45) (end 177.75 56.35) (width 0.2) (layer "B.Cu") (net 15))
 (segment (start 173.75 83.475) (end 173.75 65.45) (width 0.2) (layer "B.Cu") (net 15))
 (segment (start 167.35 83.475) (end 173.75 83.475) (width 0.2) (layer "B.Cu") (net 15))
 (segment (start 177.75 56.35) (end 177.51 56.11) (width 0.2) (layer "B.Cu") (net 15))
 (segment (start 160.49625 90.32875) (end 167.35 83.475) (width 0.2) (layer "B.Cu") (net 15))
 (segment (start 177.51 56.11) (end 174.47 56.11) (width 0.2) (layer "B.Cu") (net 15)))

